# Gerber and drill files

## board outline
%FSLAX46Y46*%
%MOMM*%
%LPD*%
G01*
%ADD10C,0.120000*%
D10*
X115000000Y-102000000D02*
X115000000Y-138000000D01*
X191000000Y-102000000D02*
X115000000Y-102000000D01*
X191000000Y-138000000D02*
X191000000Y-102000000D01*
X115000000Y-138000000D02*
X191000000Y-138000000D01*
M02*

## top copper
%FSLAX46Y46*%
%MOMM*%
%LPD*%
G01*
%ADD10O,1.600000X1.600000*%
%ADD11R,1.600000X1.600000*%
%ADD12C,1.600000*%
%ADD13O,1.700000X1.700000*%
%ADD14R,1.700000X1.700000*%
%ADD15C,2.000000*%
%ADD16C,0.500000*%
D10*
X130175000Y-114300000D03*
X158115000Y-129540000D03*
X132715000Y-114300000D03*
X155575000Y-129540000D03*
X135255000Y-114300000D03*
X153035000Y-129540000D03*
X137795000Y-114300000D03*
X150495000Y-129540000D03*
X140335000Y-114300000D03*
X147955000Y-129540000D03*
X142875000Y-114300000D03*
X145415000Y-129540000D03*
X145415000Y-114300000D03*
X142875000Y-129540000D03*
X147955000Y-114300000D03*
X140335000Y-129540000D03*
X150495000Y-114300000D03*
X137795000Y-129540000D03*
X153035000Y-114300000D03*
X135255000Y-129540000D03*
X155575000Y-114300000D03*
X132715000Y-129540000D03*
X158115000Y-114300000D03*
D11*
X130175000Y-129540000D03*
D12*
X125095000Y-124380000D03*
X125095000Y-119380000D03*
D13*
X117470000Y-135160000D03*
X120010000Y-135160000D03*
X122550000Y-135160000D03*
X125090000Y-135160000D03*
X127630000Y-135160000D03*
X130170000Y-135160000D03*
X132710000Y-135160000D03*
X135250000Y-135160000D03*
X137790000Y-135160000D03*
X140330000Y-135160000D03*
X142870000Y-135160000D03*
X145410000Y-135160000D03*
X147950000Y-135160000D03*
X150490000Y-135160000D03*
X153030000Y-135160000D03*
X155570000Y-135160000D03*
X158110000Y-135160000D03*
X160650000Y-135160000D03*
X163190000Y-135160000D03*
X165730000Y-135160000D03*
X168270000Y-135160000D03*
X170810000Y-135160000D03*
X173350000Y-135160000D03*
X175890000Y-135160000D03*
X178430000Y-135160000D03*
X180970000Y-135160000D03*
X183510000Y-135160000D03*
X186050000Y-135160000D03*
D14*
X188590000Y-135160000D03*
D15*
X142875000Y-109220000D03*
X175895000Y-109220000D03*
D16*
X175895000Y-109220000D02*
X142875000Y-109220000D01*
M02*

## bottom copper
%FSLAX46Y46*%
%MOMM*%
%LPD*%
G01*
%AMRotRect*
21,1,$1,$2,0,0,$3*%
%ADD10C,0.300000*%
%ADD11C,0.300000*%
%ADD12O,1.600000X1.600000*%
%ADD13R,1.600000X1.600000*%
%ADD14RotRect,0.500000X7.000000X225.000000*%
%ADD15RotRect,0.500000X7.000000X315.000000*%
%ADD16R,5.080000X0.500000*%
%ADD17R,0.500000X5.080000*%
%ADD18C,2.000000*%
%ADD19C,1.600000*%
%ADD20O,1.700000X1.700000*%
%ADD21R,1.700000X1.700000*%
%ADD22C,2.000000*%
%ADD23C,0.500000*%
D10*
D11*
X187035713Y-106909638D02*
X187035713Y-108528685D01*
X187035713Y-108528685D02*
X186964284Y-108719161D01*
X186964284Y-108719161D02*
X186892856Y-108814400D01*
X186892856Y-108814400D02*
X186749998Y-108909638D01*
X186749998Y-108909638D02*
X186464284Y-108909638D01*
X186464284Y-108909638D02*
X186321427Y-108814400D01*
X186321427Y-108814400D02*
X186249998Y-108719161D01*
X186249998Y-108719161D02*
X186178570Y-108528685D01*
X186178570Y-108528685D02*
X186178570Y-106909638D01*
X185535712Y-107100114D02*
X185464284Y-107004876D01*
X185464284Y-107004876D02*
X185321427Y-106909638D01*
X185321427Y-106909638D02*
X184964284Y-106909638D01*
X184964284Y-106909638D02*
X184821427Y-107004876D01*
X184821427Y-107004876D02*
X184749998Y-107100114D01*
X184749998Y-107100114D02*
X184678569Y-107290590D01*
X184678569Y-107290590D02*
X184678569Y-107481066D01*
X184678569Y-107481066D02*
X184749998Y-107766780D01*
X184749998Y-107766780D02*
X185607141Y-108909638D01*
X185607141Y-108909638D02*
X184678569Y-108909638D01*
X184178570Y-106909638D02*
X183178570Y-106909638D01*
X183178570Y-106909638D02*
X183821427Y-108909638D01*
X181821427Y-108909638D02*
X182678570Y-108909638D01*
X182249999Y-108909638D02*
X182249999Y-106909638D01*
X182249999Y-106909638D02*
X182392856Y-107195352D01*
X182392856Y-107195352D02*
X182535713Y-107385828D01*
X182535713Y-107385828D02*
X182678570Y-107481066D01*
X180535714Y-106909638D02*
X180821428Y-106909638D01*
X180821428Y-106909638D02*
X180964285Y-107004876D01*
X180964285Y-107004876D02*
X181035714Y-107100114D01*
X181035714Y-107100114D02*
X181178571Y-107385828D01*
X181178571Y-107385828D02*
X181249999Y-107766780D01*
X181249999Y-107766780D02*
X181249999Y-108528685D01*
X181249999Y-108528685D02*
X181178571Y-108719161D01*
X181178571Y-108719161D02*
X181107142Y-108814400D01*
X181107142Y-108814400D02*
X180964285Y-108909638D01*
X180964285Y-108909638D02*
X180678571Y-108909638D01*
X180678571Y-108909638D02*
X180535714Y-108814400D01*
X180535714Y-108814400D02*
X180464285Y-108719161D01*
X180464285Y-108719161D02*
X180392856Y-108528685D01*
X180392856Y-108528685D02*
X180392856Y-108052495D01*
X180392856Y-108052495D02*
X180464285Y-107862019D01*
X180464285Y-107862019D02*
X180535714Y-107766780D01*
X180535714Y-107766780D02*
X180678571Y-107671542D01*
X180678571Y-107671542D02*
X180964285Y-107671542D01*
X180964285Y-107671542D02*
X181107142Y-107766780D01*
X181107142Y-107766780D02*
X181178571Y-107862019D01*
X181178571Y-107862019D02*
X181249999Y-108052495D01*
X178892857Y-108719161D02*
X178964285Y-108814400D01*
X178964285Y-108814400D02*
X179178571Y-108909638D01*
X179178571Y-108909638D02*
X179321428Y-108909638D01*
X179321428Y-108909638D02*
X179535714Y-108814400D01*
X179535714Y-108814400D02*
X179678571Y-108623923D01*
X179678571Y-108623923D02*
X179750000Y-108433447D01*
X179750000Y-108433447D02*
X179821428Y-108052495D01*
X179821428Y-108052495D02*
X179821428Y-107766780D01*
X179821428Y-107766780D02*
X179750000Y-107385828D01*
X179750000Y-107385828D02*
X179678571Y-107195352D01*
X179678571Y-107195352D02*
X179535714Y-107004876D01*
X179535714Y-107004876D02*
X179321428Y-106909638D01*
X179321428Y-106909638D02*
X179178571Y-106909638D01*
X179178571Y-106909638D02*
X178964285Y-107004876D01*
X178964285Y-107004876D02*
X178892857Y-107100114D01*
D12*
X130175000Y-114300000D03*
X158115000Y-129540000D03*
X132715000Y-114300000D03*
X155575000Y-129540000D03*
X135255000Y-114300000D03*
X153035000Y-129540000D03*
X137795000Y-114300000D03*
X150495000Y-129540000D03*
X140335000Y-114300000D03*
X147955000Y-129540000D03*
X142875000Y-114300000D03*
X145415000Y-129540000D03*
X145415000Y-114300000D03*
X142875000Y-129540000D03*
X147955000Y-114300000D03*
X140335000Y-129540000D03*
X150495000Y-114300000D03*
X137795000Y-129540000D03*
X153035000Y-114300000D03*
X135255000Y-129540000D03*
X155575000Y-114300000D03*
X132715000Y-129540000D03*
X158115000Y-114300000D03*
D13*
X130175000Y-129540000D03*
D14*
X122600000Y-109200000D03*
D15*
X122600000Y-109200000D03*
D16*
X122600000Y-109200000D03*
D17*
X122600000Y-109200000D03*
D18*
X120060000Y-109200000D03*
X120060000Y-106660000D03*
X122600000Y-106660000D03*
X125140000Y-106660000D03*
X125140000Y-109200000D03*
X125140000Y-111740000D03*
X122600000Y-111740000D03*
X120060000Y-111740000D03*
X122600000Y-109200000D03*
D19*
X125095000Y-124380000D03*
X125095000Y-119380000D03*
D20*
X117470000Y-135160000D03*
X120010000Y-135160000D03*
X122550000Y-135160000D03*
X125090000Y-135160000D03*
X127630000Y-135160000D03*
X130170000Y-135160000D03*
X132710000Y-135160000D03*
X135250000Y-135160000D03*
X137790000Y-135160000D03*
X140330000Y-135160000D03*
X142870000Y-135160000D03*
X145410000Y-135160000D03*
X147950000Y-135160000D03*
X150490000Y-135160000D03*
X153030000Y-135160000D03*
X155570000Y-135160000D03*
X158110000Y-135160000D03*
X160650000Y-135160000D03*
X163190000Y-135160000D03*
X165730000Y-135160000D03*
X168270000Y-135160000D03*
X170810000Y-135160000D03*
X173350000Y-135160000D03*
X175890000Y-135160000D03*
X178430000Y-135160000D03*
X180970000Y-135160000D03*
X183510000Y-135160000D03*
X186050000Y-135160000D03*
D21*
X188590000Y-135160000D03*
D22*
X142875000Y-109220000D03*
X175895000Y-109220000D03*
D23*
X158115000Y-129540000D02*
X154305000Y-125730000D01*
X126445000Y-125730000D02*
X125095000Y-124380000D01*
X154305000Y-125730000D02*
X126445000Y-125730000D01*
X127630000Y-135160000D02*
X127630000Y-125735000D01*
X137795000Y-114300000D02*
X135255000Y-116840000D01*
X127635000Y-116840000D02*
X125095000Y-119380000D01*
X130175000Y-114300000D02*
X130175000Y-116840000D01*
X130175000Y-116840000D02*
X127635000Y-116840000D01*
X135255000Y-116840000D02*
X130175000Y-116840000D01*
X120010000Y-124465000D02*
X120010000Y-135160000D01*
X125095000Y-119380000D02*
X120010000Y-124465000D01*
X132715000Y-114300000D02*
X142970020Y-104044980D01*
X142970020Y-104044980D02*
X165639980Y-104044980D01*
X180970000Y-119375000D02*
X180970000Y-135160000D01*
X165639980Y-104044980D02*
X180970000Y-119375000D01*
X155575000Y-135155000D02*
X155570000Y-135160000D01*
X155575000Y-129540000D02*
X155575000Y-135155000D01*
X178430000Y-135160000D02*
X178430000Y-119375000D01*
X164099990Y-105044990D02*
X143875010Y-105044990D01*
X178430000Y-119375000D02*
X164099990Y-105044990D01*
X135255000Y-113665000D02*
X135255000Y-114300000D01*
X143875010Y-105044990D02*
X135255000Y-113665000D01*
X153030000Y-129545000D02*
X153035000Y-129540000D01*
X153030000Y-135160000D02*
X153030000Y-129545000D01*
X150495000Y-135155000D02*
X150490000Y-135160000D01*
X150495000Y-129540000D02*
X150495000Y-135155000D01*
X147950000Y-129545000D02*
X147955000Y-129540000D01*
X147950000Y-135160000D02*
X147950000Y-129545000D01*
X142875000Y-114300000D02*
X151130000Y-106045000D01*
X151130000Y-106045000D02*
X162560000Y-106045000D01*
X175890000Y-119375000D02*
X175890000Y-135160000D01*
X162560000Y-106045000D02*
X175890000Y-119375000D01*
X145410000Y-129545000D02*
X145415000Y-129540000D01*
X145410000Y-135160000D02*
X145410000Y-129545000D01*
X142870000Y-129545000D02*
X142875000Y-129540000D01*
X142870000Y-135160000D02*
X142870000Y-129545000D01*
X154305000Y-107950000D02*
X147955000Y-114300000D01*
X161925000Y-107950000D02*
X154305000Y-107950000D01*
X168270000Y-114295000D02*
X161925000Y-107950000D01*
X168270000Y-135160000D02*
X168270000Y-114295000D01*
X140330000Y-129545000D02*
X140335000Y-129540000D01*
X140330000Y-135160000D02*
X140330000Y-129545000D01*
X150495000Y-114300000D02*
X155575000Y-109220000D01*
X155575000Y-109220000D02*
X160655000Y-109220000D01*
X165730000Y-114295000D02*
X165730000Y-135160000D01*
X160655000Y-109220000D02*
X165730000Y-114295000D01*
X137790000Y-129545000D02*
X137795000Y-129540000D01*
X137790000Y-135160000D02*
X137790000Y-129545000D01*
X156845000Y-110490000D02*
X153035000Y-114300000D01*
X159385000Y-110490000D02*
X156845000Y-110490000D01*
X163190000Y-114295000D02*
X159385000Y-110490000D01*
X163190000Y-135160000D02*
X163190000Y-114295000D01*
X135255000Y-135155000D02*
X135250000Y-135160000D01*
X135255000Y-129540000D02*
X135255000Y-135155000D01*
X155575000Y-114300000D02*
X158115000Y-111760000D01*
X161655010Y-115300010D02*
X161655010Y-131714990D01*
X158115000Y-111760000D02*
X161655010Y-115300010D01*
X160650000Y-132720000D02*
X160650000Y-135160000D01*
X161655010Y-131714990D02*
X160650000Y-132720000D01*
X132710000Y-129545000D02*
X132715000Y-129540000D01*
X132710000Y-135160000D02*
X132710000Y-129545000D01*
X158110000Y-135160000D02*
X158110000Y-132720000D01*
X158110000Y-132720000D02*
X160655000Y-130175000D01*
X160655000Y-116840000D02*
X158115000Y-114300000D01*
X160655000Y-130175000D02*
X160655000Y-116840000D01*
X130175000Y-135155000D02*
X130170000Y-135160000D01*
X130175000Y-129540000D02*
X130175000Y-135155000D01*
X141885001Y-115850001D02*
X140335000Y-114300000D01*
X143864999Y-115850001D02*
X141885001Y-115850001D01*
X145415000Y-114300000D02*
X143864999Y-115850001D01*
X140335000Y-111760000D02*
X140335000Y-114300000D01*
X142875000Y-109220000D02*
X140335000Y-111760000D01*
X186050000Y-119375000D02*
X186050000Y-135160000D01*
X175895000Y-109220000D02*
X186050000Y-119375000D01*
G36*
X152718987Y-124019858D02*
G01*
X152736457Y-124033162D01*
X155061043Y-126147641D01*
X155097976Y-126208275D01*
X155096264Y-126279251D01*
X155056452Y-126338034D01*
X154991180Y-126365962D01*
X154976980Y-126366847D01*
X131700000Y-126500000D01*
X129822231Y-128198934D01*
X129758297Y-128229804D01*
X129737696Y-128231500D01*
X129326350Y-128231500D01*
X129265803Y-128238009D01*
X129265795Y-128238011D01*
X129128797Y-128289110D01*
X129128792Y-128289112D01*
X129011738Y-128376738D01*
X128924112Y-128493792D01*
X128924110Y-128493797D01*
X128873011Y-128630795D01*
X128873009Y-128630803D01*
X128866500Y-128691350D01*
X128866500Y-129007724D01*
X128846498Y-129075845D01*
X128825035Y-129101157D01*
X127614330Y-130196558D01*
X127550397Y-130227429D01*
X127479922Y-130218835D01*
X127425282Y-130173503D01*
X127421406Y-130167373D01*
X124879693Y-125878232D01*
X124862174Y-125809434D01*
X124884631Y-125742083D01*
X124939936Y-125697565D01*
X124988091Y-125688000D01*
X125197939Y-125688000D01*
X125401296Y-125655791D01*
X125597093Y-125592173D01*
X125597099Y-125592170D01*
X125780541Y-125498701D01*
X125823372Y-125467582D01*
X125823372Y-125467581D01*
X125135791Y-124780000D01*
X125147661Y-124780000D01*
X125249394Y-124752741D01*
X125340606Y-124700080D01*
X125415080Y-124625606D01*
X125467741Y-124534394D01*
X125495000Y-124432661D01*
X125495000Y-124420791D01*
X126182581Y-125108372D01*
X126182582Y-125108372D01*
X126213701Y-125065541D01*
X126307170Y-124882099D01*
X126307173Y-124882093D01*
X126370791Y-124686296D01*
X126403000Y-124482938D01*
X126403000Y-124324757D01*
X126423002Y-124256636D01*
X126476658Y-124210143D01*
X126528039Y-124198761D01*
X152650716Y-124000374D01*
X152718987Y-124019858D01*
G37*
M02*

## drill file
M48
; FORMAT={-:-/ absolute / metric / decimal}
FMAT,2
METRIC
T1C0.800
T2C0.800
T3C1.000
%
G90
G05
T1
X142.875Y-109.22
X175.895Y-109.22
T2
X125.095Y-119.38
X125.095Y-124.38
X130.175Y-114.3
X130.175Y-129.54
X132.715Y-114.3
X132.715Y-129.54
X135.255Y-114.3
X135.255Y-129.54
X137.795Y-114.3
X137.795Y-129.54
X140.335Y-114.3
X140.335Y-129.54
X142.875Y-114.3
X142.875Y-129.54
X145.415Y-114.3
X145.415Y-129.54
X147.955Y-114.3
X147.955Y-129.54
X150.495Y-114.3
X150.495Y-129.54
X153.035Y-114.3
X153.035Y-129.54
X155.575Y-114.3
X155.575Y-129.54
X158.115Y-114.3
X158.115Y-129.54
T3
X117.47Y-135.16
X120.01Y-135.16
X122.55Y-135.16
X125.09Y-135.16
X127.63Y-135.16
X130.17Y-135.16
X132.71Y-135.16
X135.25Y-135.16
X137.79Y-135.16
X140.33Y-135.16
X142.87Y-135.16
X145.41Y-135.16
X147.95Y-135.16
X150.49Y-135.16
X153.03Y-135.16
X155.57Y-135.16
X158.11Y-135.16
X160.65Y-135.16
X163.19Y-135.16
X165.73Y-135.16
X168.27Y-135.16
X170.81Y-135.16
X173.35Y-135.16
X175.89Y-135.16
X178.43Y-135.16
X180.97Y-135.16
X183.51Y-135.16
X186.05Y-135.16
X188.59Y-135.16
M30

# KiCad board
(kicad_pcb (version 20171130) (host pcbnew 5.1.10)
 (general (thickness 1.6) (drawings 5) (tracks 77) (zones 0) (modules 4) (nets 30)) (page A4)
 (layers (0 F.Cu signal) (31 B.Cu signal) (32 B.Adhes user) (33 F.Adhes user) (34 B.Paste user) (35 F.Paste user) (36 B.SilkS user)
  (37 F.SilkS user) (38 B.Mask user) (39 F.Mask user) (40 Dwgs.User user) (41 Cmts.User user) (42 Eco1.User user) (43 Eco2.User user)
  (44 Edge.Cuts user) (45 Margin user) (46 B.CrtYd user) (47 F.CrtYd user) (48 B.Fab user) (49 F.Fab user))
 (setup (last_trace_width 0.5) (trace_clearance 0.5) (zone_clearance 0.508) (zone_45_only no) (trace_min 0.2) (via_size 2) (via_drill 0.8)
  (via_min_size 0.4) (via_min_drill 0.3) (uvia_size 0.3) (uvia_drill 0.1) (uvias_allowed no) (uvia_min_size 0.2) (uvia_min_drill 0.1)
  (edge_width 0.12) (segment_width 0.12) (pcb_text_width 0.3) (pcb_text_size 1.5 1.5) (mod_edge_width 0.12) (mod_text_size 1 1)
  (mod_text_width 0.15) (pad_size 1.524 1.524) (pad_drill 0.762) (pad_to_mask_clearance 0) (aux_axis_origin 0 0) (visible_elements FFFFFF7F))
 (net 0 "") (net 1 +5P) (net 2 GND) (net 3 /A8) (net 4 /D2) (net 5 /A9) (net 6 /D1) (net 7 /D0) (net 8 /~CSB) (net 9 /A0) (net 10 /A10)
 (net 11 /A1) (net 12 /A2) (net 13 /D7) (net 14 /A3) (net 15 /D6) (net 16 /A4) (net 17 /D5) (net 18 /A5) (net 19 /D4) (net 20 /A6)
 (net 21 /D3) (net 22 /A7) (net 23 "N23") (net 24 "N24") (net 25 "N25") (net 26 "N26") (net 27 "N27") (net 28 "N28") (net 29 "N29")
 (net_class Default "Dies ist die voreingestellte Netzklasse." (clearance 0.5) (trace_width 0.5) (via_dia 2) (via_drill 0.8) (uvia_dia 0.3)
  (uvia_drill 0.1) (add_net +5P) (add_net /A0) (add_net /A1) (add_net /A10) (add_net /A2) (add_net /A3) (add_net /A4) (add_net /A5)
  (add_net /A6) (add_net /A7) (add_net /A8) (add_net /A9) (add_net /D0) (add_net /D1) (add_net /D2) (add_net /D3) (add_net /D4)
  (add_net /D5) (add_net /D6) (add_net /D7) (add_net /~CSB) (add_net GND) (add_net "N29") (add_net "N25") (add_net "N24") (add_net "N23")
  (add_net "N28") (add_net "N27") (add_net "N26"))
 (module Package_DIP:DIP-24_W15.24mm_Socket (layer F.Cu) (at 130.175 129.54 90)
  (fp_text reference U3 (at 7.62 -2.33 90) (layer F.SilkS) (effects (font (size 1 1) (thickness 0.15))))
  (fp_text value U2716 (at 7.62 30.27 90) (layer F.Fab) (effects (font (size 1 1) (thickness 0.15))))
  (pad 24 thru_hole oval (at 15.24 0 90) (size 1.6 1.6) (drill 0.8) (layers *.Cu *.Mask) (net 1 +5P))
  (pad 12 thru_hole oval (at 0 27.94 90) (size 1.6 1.6) (drill 0.8) (layers *.Cu *.Mask) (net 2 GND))
  (pad 23 thru_hole oval (at 15.24 2.54 90) (size 1.6 1.6) (drill 0.8) (layers *.Cu *.Mask) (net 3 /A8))
  (pad 11 thru_hole oval (at 0 25.4 90) (size 1.6 1.6) (drill 0.8) (layers *.Cu *.Mask) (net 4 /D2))
  (pad 22 thru_hole oval (at 15.24 5.08 90) (size 1.6 1.6) (drill 0.8) (layers *.Cu *.Mask) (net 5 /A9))
  (pad 10 thru_hole oval (at 0 22.86 90) (size 1.6 1.6) (drill 0.8) (layers *.Cu *.Mask) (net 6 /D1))
  (pad 21 thru_hole oval (at 15.24 7.62 90) (size 1.6 1.6) (drill 0.8) (layers *.Cu *.Mask) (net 1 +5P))
  (pad 9 thru_hole oval (at 0 20.32 90) (size 1.6 1.6) (drill 0.8) (layers *.Cu *.Mask) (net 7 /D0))
  (pad 20 thru_hole oval (at 15.24 10.16 90) (size 1.6 1.6) (drill 0.8) (layers *.Cu *.Mask) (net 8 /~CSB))
  (pad 8 thru_hole oval (at 0 17.78 90) (size 1.6 1.6) (drill 0.8) (layers *.Cu *.Mask) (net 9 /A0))
  (pad 19 thru_hole oval (at 15.24 12.7 90) (size 1.6 1.6) (drill 0.8) (layers *.Cu *.Mask) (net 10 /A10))
  (pad 7 thru_hole oval (at 0 15.24 90) (size 1.6 1.6) (drill 0.8) (layers *.Cu *.Mask) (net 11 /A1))
  (pad 18 thru_hole oval (at 15.24 15.24 90) (size 1.6 1.6) (drill 0.8) (layers *.Cu *.Mask) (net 8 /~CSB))
  (pad 6 thru_hole oval (at 0 12.7 90) (size 1.6 1.6) (drill 0.8) (layers *.Cu *.Mask) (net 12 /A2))
  (pad 17 thru_hole oval (at 15.24 17.78 90) (size 1.6 1.6) (drill 0.8) (layers *.Cu *.Mask) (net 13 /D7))
  (pad 5 thru_hole oval (at 0 10.16 90) (size 1.6 1.6) (drill 0.8) (layers *.Cu *.Mask) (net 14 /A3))
  (pad 16 thru_hole oval (at 15.24 20.32 90) (size 1.6 1.6) (drill 0.8) (layers *.Cu *.Mask) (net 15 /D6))
  (pad 4 thru_hole oval (at 0 7.62 90) (size 1.6 1.6) (drill 0.8) (layers *.Cu *.Mask) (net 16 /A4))
  (pad 15 thru_hole oval (at 15.24 22.86 90) (size 1.6 1.6) (drill 0.8) (layers *.Cu *.Mask) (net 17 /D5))
  (pad 3 thru_hole oval (at 0 5.08 90) (size 1.6 1.6) (drill 0.8) (layers *.Cu *.Mask) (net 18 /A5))
  (pad 14 thru_hole oval (at 15.24 25.4 90) (size 1.6 1.6) (drill 0.8) (layers *.Cu *.Mask) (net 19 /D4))
  (pad 2 thru_hole oval (at 0 2.54 90) (size 1.6 1.6) (drill 0.8) (layers *.Cu *.Mask) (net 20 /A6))
  (pad 13 thru_hole oval (at 15.24 27.94 90) (size 1.6 1.6) (drill 0.8) (layers *.Cu *.Mask) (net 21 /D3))
  (pad 1 thru_hole rect (at 0 0 90) (size 1.6 1.6) (drill 0.8) (layers *.Cu *.Mask) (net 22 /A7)))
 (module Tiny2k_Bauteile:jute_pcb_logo (layer B.Cu) (at 122.6 109.2)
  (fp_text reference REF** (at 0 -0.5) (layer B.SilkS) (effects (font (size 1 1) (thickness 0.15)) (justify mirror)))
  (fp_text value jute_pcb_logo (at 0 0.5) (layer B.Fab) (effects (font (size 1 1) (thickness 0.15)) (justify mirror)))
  (pad 2 smd rect (at 0 0 225) (size 0.5 7) (layers B.Cu B.Paste B.Mask))
  (pad 2 smd rect (at 0 0 315) (size 0.5 7) (layers B.Cu B.Paste B.Mask))
  (pad 2 smd rect (at 0 0 270) (size 0.5 5.08) (layers B.Cu B.Paste B.Mask))
  (pad 2 smd rect (at 0 0) (size 0.5 5.08) (layers B.Cu B.Paste B.Mask))
  (pad 1 smd circle (at -2.54 0) (size 2 2) (layers B.Cu B.Paste B.Mask))
  (pad 1 smd circle (at -2.54 -2.54) (size 2 2) (layers B.Cu B.Paste B.Mask))
  (pad 1 smd circle (at 0 -2.54) (size 2 2) (layers B.Cu B.Paste B.Mask))
  (pad 1 smd circle (at 2.54 -2.54) (size 2 2) (layers B.Cu B.Paste B.Mask))
  (pad 1 smd circle (at 2.54 0) (size 2 2) (layers B.Cu B.Paste B.Mask))
  (pad 1 smd circle (at 2.54 2.54) (size 2 2) (layers B.Cu B.Paste B.Mask))
  (pad 1 smd circle (at 0 2.54) (size 2 2) (layers B.Cu B.Paste B.Mask))
  (pad 1 smd circle (at -2.54 2.54) (size 2 2) (layers B.Cu B.Paste B.Mask))
  (pad 1 smd circle (at 0 0) (size 2 2) (layers B.Cu B.Paste B.Mask)))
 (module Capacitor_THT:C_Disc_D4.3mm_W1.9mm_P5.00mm (layer F.Cu) (at 125.095 119.38 270)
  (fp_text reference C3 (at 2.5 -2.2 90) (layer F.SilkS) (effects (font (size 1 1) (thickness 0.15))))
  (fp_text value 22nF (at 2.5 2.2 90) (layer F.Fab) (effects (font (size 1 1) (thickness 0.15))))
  (pad 2 thru_hole circle (at 5 0 270) (size 1.6 1.6) (drill 0.8) (layers *.Cu *.Mask) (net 2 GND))
  (pad 1 thru_hole circle (at 0 0 270) (size 1.6 1.6) (drill 0.8) (layers *.Cu *.Mask) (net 1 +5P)))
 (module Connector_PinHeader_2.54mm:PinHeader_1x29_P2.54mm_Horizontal (layer F.Cu) (at 188.59 135.16 270)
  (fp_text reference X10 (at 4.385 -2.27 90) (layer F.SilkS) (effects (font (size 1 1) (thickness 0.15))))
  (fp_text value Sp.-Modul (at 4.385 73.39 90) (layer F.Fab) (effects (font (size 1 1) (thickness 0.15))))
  (pad 29 thru_hole oval (at 0 71.12 270) (size 1.7 1.7) (drill 1) (layers *.Cu *.Mask) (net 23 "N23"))
  (pad 28 thru_hole oval (at 0 68.58 270) (size 1.7 1.7) (drill 1) (layers *.Cu *.Mask) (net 1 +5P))
  (pad 27 thru_hole oval (at 0 66.04 270) (size 1.7 1.7) (drill 1) (layers *.Cu *.Mask) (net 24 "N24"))
  (pad 26 thru_hole oval (at 0 63.5 270) (size 1.7 1.7) (drill 1) (layers *.Cu *.Mask) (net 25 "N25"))
  (pad 25 thru_hole oval (at 0 60.96 270) (size 1.7 1.7) (drill 1) (layers *.Cu *.Mask) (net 2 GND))
  (pad 24 thru_hole oval (at 0 58.42 270) (size 1.7 1.7) (drill 1) (layers *.Cu *.Mask) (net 22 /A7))
  (pad 23 thru_hole oval (at 0 55.88 270) (size 1.7 1.7) (drill 1) (layers *.Cu *.Mask) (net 20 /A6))
  (pad 22 thru_hole oval (at 0 53.34 270) (size 1.7 1.7) (drill 1) (layers *.Cu *.Mask) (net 18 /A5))
  (pad 21 thru_hole oval (at 0 50.8 270) (size 1.7 1.7) (drill 1) (layers *.Cu *.Mask) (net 16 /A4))
  (pad 20 thru_hole oval (at 0 48.26 270) (size 1.7 1.7) (drill 1) (layers *.Cu *.Mask) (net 14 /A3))
  (pad 19 thru_hole oval (at 0 45.72 270) (size 1.7 1.7) (drill 1) (layers *.Cu *.Mask) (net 12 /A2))
  (pad 18 thru_hole oval (at 0 43.18 270) (size 1.7 1.7) (drill 1) (layers *.Cu *.Mask) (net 11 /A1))
  (pad 17 thru_hole oval (at 0 40.64 270) (size 1.7 1.7) (drill 1) (layers *.Cu *.Mask) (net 9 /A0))
  (pad 16 thru_hole oval (at 0 38.1 270) (size 1.7 1.7) (drill 1) (layers *.Cu *.Mask) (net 7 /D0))
  (pad 15 thru_hole oval (at 0 35.56 270) (size 1.7 1.7) (drill 1) (layers *.Cu *.Mask) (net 6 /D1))
  (pad 14 thru_hole oval (at 0 33.02 270) (size 1.7 1.7) (drill 1) (layers *.Cu *.Mask) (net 4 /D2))
  (pad 13 thru_hole oval (at 0 30.48 270) (size 1.7 1.7) (drill 1) (layers *.Cu *.Mask) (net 21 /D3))
  (pad 12 thru_hole oval (at 0 27.94 270) (size 1.7 1.7) (drill 1) (layers *.Cu *.Mask) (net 19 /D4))
  (pad 11 thru_hole oval (at 0 25.4 270) (size 1.7 1.7) (drill 1) (layers *.Cu *.Mask) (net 17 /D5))
  (pad 10 thru_hole oval (at 0 22.86 270) (size 1.7 1.7) (drill 1) (layers *.Cu *.Mask) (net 15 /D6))
  (pad 9 thru_hole oval (at 0 20.32 270) (size 1.7 1.7) (drill 1) (layers *.Cu *.Mask) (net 13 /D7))
  (pad 8 thru_hole oval (at 0 17.78 270) (size 1.7 1.7) (drill 1) (layers *.Cu *.Mask) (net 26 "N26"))
  (pad 7 thru_hole oval (at 0 15.24 270) (size 1.7 1.7) (drill 1) (layers *.Cu *.Mask) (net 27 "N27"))
  (pad 6 thru_hole oval (at 0 12.7 270) (size 1.7 1.7) (drill 1) (layers *.Cu *.Mask) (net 10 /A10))
  (pad 5 thru_hole oval (at 0 10.16 270) (size 1.7 1.7) (drill 1) (layers *.Cu *.Mask) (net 5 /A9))
  (pad 4 thru_hole oval (at 0 7.62 270) (size 1.7 1.7) (drill 1) (layers *.Cu *.Mask) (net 3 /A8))
  (pad 3 thru_hole oval (at 0 5.08 270) (size 1.7 1.7) (drill 1) (layers *.Cu *.Mask) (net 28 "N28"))
  (pad 2 thru_hole oval (at 0 2.54 270) (size 1.7 1.7) (drill 1) (layers *.Cu *.Mask) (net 8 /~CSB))
  (pad 1 thru_hole rect (at 0 0 270) (size 1.7 1.7) (drill 1) (layers *.Cu *.Mask) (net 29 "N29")))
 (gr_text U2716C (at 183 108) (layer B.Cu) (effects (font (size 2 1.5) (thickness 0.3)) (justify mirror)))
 (gr_line (start 115 102) (end 115 138) (layer Edge.Cuts) (width 0.12))
 (gr_line (start 191 102) (end 115 102) (layer Edge.Cuts) (width 0.12))
 (gr_line (start 191 138) (end 191 102) (layer Edge.Cuts) (width 0.12))
 (gr_line (start 115 138) (end 191 138) (layer Edge.Cuts) (width 0.12))
 (segment (start 158.115 129.54) (end 154.305 125.73) (width 0.5) (layer B.Cu) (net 2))
 (segment (start 126.445 125.73) (end 125.095 124.38) (width 0.5) (layer B.Cu) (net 2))
 (segment (start 154.305 125.73) (end 126.445 125.73) (width 0.5) (layer B.Cu) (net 2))
 (segment (start 127.63 135.16) (end 127.63 125.735) (width 0.5) (layer B.Cu) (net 2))
 (segment (start 137.795 114.3) (end 135.255 116.84) (width 0.5) (layer B.Cu) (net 1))
 (segment (start 127.635 116.84) (end 125.095 119.38) (width 0.5) (layer B.Cu) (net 1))
 (segment (start 130.175 114.3) (end 130.175 116.84) (width 0.5) (layer B.Cu) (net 1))
 (segment (start 130.175 116.84) (end 127.635 116.84) (width 0.5) (layer B.Cu) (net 1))
 (segment (start 135.255 116.84) (end 130.175 116.84) (width 0.5) (layer B.Cu) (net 1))
 (segment (start 120.01 124.465) (end 120.01 135.16) (width 0.5) (layer B.Cu) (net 1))
 (segment (start 125.095 119.38) (end 120.01 124.465) (width 0.5) (layer B.Cu) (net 1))
 (segment (start 132.715 114.3) (end 142.97002 104.04498) (width 0.5) (layer B.Cu) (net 3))
 (segment (start 142.97002 104.04498) (end 165.63998 104.04498) (width 0.5) (layer B.Cu) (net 3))
 (segment (start 180.97 119.375) (end 180.97 135.16) (width 0.5) (layer B.Cu) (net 3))
 (segment (start 165.63998 104.04498) (end 180.97 119.375) (width 0.5) (layer B.Cu) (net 3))
 (segment (start 155.575 135.155) (end 155.57 135.16) (width 0.5) (layer B.Cu) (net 4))
 (segment (start 155.575 129.54) (end 155.575 135.155) (width 0.5) (layer B.Cu) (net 4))
 (segment (start 178.43 135.16) (end 178.43 119.375) (width 0.5) (layer B.Cu) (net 5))
 (segment (start 164.09999 105.04499) (end 143.87501 105.04499) (width 0.5) (layer B.Cu) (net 5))
 (segment (start 178.43 119.375) (end 164.09999 105.04499) (width 0.5) (layer B.Cu) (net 5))
 (segment (start 135.255 113.665) (end 135.255 114.3) (width 0.5) (layer B.Cu) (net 5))
 (segment (start 143.87501 105.04499) (end 135.255 113.665) (width 0.5) (layer B.Cu) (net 5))
 (segment (start 153.03 129.545) (end 153.035 129.54) (width 0.5) (layer B.Cu) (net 6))
 (segment (start 153.03 135.16) (end 153.03 129.545) (width 0.5) (layer B.Cu) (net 6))
 (segment (start 150.495 135.155) (end 150.49 135.16) (width 0.5) (layer B.Cu) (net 7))
 (segment (start 150.495 129.54) (end 150.495 135.155) (width 0.5) (layer B.Cu) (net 7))
 (segment (start 147.95 129.545) (end 147.955 129.54) (width 0.5) (layer B.Cu) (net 9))
 (segment (start 147.95 135.16) (end 147.95 129.545) (width 0.5) (layer B.Cu) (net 9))
 (segment (start 142.875 114.3) (end 151.13 106.045) (width 0.5) (layer B.Cu) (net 10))
 (segment (start 151.13 106.045) (end 162.56 106.045) (width 0.5) (layer B.Cu) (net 10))
 (segment (start 175.89 119.375) (end 175.89 135.16) (width 0.5) (layer B.Cu) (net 10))
 (segment (start 162.56 106.045) (end 175.89 119.375) (width 0.5) (layer B.Cu) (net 10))
 (segment (start 145.41 129.545) (end 145.415 129.54) (width 0.5) (layer B.Cu) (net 11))
 (segment (start 145.41 135.16) (end 145.41 129.545) (width 0.5) (layer B.Cu) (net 11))
 (segment (start 142.87 129.545) (end 142.875 129.54) (width 0.5) (layer B.Cu) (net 12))
 (segment (start 142.87 135.16) (end 142.87 129.545) (width 0.5) (layer B.Cu) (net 12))
 (segment (start 154.305 107.95) (end 147.955 114.3) (width 0.5) (layer B.Cu) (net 13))
 (segment (start 161.925 107.95) (end 154.305 107.95) (width 0.5) (layer B.Cu) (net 13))
 (segment (start 168.27 114.295) (end 161.925 107.95) (width 0.5) (layer B.Cu) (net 13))
 (segment (start 168.27 135.16) (end 168.27 114.295) (width 0.5) (layer B.Cu) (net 13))
 (segment (start 140.33 129.545) (end 140.335 129.54) (width 0.5) (layer B.Cu) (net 14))
 (segment (start 140.33 135.16) (end 140.33 129.545) (width 0.5) (layer B.Cu) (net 14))
 (segment (start 150.495 114.3) (end 155.575 109.22) (width 0.5) (layer B.Cu) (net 15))
 (segment (start 155.575 109.22) (end 160.655 109.22) (width 0.5) (layer B.Cu) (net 15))
 (segment (start 165.73 114.295) (end 165.73 135.16) (width 0.5) (layer B.Cu) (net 15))
 (segment (start 160.655 109.22) (end 165.73 114.295) (width 0.5) (layer B.Cu) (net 15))
 (segment (start 137.79 129.545) (end 137.795 129.54) (width 0.5) (layer B.Cu) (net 16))
 (segment (start 137.79 135.16) (end 137.79 129.545) (width 0.5) (layer B.Cu) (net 16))
 (segment (start 156.845 110.49) (end 153.035 114.3) (width 0.5) (layer B.Cu) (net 17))
 (segment (start 159.385 110.49) (end 156.845 110.49) (width 0.5) (layer B.Cu) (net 17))
 (segment (start 163.19 114.295) (end 159.385 110.49) (width 0.5) (layer B.Cu) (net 17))
 (segment (start 163.19 135.16) (end 163.19 114.295) (width 0.5) (layer B.Cu) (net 17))
 (segment (start 135.255 135.155) (end 135.25 135.16) (width 0.5) (layer B.Cu) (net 18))
 (segment (start 135.255 129.54) (end 135.255 135.155) (width 0.5) (layer B.Cu) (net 18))
 (segment (start 155.575 114.3) (end 158.115 111.76) (width 0.5) (layer B.Cu) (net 19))
 (segment (start 161.65501 115.30001) (end 161.65501 131.71499) (width 0.5) (layer B.Cu) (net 19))
 (segment (start 158.115 111.76) (end 161.65501 115.30001) (width 0.5) (layer B.Cu) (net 19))
 (segment (start 160.65 132.72) (end 160.65 135.16) (width 0.5) (layer B.Cu) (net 19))
 (segment (start 161.65501 131.71499) (end 160.65 132.72) (width 0.5) (layer B.Cu) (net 19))
 (segment (start 132.71 129.545) (end 132.715 129.54) (width 0.5) (layer B.Cu) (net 20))
 (segment (start 132.71 135.16) (end 132.71 129.545) (width 0.5) (layer B.Cu) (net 20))
 (segment (start 158.11 135.16) (end 158.11 132.72) (width 0.5) (layer B.Cu) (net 21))
 (segment (start 158.11 132.72) (end 160.655 130.175) (width 0.5) (layer B.Cu) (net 21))
 (segment (start 160.655 116.84) (end 158.115 114.3) (width 0.5) (layer B.Cu) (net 21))
 (segment (start 160.655 130.175) (end 160.655 116.84) (width 0.5) (layer B.Cu) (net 21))
 (segment (start 130.175 135.155) (end 130.17 135.16) (width 0.5) (layer B.Cu) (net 22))
 (segment (start 130.175 129.54) (end 130.175 135.155) (width 0.5) (layer B.Cu) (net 22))
 (segment (start 141.885001 115.850001) (end 140.335 114.3) (width 0.5) (layer B.Cu) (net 8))
 (segment (start 143.864999 115.850001) (end 141.885001 115.850001) (width 0.5) (layer B.Cu) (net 8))
 (segment (start 145.415 114.3) (end 143.864999 115.850001) (width 0.5) (layer B.Cu) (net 8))
 (via (at 142.875 109.22) (size 2) (drill 0.8) (layers F.Cu B.Cu) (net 8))
 (segment (start 140.335 111.76) (end 140.335 114.3) (width 0.5) (layer B.Cu) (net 8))
 (segment (start 142.875 109.22) (end 140.335 111.76) (width 0.5) (layer B.Cu) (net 8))
 (segment (start 186.05 119.375) (end 186.05 135.16) (width 0.5) (layer B.Cu) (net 8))
 (segment (start 175.895 109.22) (end 186.05 119.375) (width 0.5) (layer B.Cu) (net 8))
 (via (at 175.895 109.22) (size 2) (drill 0.8) (layers F.Cu B.Cu) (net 8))
 (segment (start 175.895 109.22) (end 142.875 109.22) (width 0.5) (layer F.Cu) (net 8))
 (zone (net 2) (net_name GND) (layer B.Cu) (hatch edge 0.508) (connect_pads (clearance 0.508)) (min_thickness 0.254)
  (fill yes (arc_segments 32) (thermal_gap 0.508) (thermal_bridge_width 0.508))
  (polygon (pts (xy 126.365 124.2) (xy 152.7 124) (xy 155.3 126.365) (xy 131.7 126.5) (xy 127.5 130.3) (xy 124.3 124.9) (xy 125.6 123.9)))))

